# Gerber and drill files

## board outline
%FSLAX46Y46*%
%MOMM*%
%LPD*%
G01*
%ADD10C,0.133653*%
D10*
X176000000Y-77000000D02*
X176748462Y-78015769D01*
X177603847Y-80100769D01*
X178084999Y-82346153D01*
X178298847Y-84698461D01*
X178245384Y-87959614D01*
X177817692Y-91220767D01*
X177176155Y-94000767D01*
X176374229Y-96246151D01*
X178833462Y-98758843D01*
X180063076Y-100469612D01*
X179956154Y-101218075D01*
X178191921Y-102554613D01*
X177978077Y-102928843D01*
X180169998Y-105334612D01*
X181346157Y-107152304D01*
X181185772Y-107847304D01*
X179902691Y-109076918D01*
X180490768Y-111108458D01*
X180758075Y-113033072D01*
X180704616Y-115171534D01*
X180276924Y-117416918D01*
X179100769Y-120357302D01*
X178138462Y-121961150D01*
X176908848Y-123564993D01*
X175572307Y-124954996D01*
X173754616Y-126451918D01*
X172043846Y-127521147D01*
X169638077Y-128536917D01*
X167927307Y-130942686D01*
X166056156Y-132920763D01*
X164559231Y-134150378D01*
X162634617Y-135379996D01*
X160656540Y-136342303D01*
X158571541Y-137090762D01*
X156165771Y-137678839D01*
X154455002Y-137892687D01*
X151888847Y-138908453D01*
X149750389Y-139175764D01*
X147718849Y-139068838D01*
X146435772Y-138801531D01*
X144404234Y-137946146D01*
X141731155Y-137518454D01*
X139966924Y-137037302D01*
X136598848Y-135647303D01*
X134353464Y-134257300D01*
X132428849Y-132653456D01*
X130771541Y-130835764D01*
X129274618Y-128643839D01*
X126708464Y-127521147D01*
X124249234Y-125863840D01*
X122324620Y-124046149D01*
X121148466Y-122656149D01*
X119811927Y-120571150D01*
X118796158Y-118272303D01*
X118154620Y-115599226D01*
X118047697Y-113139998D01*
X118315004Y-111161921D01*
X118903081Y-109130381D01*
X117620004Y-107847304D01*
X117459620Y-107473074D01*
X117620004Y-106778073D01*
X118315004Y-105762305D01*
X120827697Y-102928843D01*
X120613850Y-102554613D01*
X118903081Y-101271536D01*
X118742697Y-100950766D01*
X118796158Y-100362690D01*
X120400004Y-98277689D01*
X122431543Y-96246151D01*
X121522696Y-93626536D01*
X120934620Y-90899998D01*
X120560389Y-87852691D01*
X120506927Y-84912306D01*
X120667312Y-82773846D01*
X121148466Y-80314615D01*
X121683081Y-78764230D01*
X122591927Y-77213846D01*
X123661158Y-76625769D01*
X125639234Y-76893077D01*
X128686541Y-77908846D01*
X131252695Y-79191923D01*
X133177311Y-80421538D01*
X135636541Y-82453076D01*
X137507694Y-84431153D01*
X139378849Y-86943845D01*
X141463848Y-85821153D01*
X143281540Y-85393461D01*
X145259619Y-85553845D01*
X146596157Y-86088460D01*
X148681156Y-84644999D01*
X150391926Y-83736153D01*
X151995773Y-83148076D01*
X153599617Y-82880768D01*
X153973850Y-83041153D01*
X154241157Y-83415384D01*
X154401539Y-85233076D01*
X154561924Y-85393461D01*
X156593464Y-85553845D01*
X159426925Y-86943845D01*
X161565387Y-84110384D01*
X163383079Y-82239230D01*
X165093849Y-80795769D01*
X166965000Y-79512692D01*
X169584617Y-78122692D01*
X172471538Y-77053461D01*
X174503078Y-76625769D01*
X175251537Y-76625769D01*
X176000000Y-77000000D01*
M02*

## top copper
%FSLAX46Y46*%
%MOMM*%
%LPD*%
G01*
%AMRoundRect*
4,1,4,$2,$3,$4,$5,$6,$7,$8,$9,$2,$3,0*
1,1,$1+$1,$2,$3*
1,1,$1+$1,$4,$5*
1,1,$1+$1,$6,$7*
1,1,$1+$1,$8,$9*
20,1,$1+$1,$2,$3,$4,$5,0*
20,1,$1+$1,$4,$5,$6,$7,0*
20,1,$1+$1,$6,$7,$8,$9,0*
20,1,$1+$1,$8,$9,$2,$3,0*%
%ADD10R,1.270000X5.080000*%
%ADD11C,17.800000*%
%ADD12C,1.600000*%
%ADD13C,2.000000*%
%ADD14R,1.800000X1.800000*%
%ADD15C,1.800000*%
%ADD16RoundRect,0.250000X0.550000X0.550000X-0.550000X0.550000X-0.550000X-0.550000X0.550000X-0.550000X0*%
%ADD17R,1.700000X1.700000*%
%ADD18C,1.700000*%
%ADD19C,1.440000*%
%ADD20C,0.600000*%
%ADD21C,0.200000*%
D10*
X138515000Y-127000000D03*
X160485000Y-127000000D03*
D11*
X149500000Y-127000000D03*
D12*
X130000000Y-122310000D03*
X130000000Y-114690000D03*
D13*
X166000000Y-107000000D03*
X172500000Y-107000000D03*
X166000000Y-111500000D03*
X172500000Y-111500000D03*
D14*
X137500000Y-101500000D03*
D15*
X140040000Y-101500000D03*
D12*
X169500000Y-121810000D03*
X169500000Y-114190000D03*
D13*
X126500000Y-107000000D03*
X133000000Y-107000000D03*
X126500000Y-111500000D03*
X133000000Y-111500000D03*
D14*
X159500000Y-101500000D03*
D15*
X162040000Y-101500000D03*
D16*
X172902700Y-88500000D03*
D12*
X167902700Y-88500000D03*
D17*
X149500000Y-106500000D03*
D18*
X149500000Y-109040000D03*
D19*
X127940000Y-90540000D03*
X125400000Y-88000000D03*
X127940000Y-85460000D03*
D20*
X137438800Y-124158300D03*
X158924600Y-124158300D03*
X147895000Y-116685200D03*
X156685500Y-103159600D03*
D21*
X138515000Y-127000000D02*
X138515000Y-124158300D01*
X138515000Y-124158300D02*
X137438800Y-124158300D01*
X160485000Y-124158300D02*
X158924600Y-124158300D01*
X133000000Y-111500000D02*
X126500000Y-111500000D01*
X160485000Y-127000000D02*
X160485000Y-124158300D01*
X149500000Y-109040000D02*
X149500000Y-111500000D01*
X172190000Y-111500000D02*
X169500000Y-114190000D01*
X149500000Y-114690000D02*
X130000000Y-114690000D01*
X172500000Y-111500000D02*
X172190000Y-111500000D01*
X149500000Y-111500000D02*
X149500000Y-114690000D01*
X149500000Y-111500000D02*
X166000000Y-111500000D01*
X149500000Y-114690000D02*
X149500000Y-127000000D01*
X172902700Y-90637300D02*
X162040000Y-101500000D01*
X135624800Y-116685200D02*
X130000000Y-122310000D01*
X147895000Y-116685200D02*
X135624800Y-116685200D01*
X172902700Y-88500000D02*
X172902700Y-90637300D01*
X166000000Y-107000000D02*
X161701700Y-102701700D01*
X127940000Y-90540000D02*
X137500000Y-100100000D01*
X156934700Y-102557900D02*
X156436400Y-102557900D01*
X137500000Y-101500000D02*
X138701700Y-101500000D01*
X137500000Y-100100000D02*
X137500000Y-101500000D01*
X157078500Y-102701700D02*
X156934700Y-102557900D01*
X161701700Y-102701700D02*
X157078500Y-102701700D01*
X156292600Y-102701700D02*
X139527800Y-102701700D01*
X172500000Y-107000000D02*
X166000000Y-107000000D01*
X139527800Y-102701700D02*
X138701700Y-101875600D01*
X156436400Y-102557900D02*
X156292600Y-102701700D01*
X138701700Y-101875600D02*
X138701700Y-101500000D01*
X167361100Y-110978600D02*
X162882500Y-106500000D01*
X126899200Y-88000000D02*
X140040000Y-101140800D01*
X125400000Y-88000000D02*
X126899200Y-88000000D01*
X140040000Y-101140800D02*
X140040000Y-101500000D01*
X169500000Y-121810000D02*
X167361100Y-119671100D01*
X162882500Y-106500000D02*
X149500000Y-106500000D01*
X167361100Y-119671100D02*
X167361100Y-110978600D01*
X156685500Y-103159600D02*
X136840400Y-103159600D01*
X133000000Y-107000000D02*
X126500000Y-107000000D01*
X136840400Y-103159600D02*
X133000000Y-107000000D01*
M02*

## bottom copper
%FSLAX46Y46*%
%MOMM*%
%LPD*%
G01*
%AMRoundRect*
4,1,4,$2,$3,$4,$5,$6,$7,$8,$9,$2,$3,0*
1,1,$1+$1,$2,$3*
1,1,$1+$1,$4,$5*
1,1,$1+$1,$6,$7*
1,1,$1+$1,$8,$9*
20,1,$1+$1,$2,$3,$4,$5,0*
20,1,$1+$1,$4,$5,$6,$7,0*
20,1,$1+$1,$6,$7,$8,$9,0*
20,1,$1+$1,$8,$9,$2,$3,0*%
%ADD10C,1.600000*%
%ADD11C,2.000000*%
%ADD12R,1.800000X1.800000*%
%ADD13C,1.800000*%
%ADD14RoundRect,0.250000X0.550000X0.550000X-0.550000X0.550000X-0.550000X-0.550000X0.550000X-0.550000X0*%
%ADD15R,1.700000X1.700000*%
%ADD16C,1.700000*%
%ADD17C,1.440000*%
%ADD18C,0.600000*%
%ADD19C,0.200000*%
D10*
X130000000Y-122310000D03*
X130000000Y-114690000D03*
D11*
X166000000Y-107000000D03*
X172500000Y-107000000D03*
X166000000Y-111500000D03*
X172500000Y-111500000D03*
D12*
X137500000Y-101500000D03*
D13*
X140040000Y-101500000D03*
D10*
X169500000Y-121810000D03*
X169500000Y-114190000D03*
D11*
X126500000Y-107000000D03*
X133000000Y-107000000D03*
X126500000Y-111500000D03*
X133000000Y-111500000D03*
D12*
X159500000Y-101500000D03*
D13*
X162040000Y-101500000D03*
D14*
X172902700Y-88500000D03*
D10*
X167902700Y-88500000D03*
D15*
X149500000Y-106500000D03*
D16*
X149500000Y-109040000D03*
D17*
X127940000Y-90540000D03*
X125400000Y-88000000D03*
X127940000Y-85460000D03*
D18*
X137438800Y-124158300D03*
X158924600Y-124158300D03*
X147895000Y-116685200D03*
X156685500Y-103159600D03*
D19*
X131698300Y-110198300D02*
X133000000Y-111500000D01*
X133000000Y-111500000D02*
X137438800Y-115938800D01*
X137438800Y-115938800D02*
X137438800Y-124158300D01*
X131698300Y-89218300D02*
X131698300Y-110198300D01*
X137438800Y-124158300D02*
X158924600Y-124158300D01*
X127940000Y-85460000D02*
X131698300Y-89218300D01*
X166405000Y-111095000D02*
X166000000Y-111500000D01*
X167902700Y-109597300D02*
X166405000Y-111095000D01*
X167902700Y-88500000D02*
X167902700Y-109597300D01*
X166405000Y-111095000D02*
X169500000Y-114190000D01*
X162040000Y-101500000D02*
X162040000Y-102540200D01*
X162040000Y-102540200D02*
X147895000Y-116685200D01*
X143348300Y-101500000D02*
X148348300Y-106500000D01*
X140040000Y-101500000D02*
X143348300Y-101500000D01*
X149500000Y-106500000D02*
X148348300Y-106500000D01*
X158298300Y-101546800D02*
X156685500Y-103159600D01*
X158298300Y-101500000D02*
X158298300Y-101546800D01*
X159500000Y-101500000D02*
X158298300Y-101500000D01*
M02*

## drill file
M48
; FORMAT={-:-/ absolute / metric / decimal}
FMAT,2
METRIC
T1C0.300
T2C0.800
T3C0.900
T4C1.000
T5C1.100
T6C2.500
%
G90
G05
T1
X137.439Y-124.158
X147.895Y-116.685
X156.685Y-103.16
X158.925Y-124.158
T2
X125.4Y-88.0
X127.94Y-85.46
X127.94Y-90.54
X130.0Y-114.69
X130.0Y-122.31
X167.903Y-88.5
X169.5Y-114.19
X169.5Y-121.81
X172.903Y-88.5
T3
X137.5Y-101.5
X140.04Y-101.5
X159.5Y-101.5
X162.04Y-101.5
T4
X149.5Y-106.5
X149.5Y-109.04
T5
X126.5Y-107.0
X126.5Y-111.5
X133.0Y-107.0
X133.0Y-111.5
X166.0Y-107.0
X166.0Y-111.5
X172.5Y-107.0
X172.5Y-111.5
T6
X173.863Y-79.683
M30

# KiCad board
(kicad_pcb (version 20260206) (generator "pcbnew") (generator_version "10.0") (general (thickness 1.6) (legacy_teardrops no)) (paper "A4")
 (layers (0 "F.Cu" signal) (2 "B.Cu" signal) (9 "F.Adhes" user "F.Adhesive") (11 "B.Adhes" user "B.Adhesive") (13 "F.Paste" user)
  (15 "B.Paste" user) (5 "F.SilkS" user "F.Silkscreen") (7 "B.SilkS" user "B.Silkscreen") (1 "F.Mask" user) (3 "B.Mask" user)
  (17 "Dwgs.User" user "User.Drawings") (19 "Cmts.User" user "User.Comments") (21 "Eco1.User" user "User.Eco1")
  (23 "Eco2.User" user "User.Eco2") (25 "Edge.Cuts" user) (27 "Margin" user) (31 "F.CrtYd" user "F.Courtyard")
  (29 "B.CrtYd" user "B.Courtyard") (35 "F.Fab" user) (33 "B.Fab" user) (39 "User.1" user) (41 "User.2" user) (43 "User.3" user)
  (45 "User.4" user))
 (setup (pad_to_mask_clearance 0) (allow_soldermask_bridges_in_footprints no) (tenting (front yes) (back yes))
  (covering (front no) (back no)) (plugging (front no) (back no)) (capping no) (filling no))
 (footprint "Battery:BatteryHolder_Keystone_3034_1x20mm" (layer "F.Cu") (at 149.5 127)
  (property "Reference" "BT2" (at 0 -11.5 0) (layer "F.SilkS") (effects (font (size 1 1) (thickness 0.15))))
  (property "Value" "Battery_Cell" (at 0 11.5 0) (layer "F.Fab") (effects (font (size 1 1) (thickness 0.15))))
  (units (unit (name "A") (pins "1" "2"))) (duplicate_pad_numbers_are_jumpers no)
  (pad "1" smd rect (at -10.985 0) (size 1.27 5.08) (layers "F.Cu" "F.Mask" "F.Paste") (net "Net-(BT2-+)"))
  (pad "1" smd rect (at 10.985 0) (size 1.27 5.08) (layers "F.Cu" "F.Mask" "F.Paste") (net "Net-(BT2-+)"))
  (pad "2" smd circle (at 0 0) (size 17.8 17.8) (layers "F.Cu" "F.Mask") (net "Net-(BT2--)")))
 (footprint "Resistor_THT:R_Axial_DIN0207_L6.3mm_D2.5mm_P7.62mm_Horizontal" (layer "F.Cu") (at 130 122.31 90)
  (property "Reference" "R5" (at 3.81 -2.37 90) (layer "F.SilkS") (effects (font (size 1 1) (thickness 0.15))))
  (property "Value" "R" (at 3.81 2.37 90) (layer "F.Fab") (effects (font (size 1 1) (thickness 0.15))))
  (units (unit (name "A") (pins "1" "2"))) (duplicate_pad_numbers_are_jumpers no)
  (pad "1" thru_hole circle (at 0 0 90) (size 1.6 1.6) (drill 0.8) (layers "*.Cu" "*.Mask") (remove_unused_layers no) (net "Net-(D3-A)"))
  (pad "2" thru_hole circle (at 7.62 0 90) (size 1.6 1.6) (drill 0.8) (layers "*.Cu" "*.Mask") (remove_unused_layers no) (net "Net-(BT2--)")))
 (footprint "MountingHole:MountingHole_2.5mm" (layer "F.Cu") (at 173.8631 79.6828)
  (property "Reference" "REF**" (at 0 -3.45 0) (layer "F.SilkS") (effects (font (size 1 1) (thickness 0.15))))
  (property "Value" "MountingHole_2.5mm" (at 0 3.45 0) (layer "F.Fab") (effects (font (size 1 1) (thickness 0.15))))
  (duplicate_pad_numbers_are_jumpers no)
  (pad "" np_thru_hole circle (at 0 0) (size 2.5 2.5) (drill 2.5) (layers "*.Mask")))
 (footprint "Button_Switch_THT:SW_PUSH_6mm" (layer "F.Cu") (at 166 107)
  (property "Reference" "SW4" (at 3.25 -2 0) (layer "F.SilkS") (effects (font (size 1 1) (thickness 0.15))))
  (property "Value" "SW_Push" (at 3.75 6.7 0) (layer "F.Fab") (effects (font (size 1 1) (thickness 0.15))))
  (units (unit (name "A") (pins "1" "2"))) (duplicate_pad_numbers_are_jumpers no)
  (pad "1" thru_hole circle (at 0 0 90) (size 2 2) (drill 1.1) (layers "*.Cu" "*.Mask") (remove_unused_layers no) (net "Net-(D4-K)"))
  (pad "1" thru_hole circle (at 6.5 0 90) (size 2 2) (drill 1.1) (layers "*.Cu" "*.Mask") (remove_unused_layers no) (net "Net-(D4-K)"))
  (pad "2" thru_hole circle (at 0 4.5 90) (size 2 2) (drill 1.1) (layers "*.Cu" "*.Mask") (remove_unused_layers no) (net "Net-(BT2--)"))
  (pad "2" thru_hole circle (at 6.5 4.5 90) (size 2 2) (drill 1.1) (layers "*.Cu" "*.Mask") (remove_unused_layers no) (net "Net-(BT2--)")))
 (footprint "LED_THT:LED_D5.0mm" (layer "F.Cu") (at 137.5 101.5)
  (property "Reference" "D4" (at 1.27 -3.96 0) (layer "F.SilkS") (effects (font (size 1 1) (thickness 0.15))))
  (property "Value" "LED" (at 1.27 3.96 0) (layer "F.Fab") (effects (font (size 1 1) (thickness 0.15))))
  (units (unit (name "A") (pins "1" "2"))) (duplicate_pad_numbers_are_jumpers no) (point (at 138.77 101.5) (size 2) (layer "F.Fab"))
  (pad "1" thru_hole rect (at 0 0) (size 1.8 1.8) (drill 0.9) (layers "*.Cu" "*.Mask") (remove_unused_layers no) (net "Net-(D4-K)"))
  (pad "2" thru_hole circle (at 2.54 0) (size 1.8 1.8) (drill 0.9) (layers "*.Cu" "*.Mask") (remove_unused_layers no) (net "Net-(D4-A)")))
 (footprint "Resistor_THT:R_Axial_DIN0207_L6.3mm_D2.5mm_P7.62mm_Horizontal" (layer "F.Cu") (at 169.5 121.81 90)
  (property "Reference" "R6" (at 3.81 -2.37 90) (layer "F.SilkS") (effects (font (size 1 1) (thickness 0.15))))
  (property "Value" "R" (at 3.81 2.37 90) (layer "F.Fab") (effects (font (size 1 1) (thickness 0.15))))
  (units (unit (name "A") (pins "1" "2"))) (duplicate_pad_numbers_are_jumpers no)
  (pad "1" thru_hole circle (at 0 0 90) (size 1.6 1.6) (drill 0.8) (layers "*.Cu" "*.Mask") (remove_unused_layers no) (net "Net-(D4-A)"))
  (pad "2" thru_hole circle (at 7.62 0 90) (size 1.6 1.6) (drill 0.8) (layers "*.Cu" "*.Mask") (remove_unused_layers no) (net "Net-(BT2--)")))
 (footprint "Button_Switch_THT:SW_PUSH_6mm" (layer "F.Cu") (at 126.5 107)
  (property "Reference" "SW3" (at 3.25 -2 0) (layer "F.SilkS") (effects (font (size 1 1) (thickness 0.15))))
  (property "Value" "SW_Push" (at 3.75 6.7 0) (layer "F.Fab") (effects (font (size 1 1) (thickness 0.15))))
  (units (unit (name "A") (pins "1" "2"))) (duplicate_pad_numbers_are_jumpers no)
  (pad "1" thru_hole circle (at 0 0 90) (size 2 2) (drill 1.1) (layers "*.Cu" "*.Mask") (remove_unused_layers no) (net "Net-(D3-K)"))
  (pad "1" thru_hole circle (at 6.5 0 90) (size 2 2) (drill 1.1) (layers "*.Cu" "*.Mask") (remove_unused_layers no) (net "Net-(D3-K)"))
  (pad "2" thru_hole circle (at 0 4.5 90) (size 2 2) (drill 1.1) (layers "*.Cu" "*.Mask") (remove_unused_layers no) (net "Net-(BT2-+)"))
  (pad "2" thru_hole circle (at 6.5 4.5 90) (size 2 2) (drill 1.1) (layers "*.Cu" "*.Mask") (remove_unused_layers no) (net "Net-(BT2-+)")))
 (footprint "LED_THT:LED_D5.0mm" (layer "F.Cu") (at 159.5 101.5)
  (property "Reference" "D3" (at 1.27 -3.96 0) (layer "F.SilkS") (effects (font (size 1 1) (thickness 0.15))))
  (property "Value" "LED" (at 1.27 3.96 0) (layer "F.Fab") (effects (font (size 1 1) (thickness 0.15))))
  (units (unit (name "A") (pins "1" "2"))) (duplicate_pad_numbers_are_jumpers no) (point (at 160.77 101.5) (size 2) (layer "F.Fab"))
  (pad "1" thru_hole rect (at 0 0) (size 1.8 1.8) (drill 0.9) (layers "*.Cu" "*.Mask") (remove_unused_layers no) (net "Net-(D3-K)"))
  (pad "2" thru_hole circle (at 2.54 0) (size 1.8 1.8) (drill 0.9) (layers "*.Cu" "*.Mask") (remove_unused_layers no) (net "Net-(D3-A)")))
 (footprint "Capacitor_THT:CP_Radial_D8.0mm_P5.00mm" (layer "B.Cu") (at 172.9027 88.5 180)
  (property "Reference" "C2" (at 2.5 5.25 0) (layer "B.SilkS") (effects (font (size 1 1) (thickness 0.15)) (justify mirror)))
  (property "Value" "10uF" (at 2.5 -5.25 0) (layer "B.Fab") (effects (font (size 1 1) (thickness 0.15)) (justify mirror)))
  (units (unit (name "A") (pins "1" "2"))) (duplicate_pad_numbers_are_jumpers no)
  (pad "1" thru_hole roundrect (at 0 0 180) (size 1.6 1.6) (drill 0.8) (layers "*.Cu" "*.Mask") (remove_unused_layers no)
   (roundrect_rratio 0.15625) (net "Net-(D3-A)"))
  (pad "2" thru_hole circle (at 5 0 180) (size 1.6 1.6) (drill 0.8) (layers "*.Cu" "*.Mask") (remove_unused_layers no) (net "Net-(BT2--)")))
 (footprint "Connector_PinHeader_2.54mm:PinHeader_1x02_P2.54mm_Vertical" (layer "B.Cu") (at 149.5 106.5 180)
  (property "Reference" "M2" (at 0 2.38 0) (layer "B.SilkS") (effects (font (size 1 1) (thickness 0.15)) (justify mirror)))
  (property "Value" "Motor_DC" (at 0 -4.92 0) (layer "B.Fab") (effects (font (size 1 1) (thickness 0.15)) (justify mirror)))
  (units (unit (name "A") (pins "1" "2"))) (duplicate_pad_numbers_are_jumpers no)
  (pad "1" thru_hole rect (at 0 0 180) (size 1.7 1.7) (drill 1) (layers "*.Cu" "*.Mask") (remove_unused_layers no) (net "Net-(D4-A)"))
  (pad "2" thru_hole circle (at 0 -2.54 180) (size 1.7 1.7) (drill 1) (layers "*.Cu" "*.Mask") (remove_unused_layers no) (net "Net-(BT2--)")))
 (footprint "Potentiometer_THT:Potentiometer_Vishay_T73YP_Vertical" (layer "B.Cu") (at 127.94 90.54 180)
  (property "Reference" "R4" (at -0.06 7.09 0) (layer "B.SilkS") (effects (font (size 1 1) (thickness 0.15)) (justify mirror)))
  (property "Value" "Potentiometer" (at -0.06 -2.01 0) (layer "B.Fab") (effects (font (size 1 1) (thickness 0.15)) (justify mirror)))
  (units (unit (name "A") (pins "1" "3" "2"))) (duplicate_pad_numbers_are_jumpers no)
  (pad "1" thru_hole circle (at 0 0 180) (size 1.44 1.44) (drill 0.8) (layers "*.Cu" "*.Mask") (remove_unused_layers no) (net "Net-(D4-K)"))
  (pad "2" thru_hole circle (at 2.54 2.54 180) (size 1.44 1.44) (drill 0.8) (layers "*.Cu" "*.Mask") (remove_unused_layers no)
   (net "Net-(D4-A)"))
  (pad "3" thru_hole circle (at 0 5.08 180) (size 1.44 1.44) (drill 0.8) (layers "*.Cu" "*.Mask") (remove_unused_layers no)
   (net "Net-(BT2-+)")))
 (gr_poly
  (pts (xy 176 77) (xy 176.748462 78.015769) (xy 177.603847 80.100769) (xy 178.084999 82.346153) (xy 178.298847 84.698461)
   (xy 178.245384 87.959614) (xy 177.817692 91.220767) (xy 177.176155 94.000767) (xy 176.374229 96.246151) (xy 178.833462 98.758843)
   (xy 180.063076 100.469612) (xy 179.956154 101.218075) (xy 178.191921 102.554613) (xy 177.978077 102.928843) (xy 180.169998 105.334612)
   (xy 181.346157 107.152304) (xy 181.185772 107.847304) (xy 179.902691 109.076918) (xy 180.490768 111.108458) (xy 180.758075 113.033072)
   (xy 180.704616 115.171534) (xy 180.276924 117.416918) (xy 179.100769 120.357302) (xy 178.138462 121.96115) (xy 176.908848 123.564993)
   (xy 175.572307 124.954996) (xy 173.754616 126.451918) (xy 172.043846 127.521147) (xy 169.638077 128.536917) (xy 167.927307 130.942686)
   (xy 166.056156 132.920763) (xy 164.559231 134.150378) (xy 162.634617 135.379996) (xy 160.65654 136.342303) (xy 158.571541 137.090762)
   (xy 156.165771 137.678839) (xy 154.455002 137.892687) (xy 151.888847 138.908453) (xy 149.750389 139.175764) (xy 147.718849 139.068838)
   (xy 146.435772 138.801531) (xy 144.404234 137.946146) (xy 141.731155 137.518454) (xy 139.966924 137.037302) (xy 136.598848 135.647303)
   (xy 134.353464 134.2573) (xy 132.428849 132.653456) (xy 130.771541 130.835764) (xy 129.274618 128.643839) (xy 126.708464 127.521147)
   (xy 124.249234 125.86384) (xy 122.32462 124.046149) (xy 121.148466 122.656149) (xy 119.811927 120.57115) (xy 118.796158 118.272303)
   (xy 118.15462 115.599226) (xy 118.047697 113.139998) (xy 118.315004 111.161921) (xy 118.903081 109.130381) (xy 117.620004 107.847304)
   (xy 117.45962 107.473074) (xy 117.620004 106.778073) (xy 118.315004 105.762305) (xy 120.827697 102.928843) (xy 120.61385 102.554613)
   (xy 118.903081 101.271536) (xy 118.742697 100.950766) (xy 118.796158 100.36269) (xy 120.400004 98.277689) (xy 122.431543 96.246151)
   (xy 121.522696 93.626536) (xy 120.93462 90.899998) (xy 120.560389 87.852691) (xy 120.506927 84.912306) (xy 120.667312 82.773846)
   (xy 121.148466 80.314615) (xy 121.683081 78.76423) (xy 122.591927 77.213846) (xy 123.661158 76.625769) (xy 125.639234 76.893077)
   (xy 128.686541 77.908846) (xy 131.252695 79.191923) (xy 133.177311 80.421538) (xy 135.636541 82.453076) (xy 137.507694 84.431153)
   (xy 139.378849 86.943845) (xy 141.463848 85.821153) (xy 143.28154 85.393461) (xy 145.259619 85.553845) (xy 146.596157 86.08846)
   (xy 148.681156 84.644999) (xy 150.391926 83.736153) (xy 151.995773 83.148076) (xy 153.599617 82.880768) (xy 153.97385 83.041153)
   (xy 154.241157 83.415384) (xy 154.401539 85.233076) (xy 154.561924 85.393461) (xy 156.593464 85.553845) (xy 159.426925 86.943845)
   (xy 161.565387 84.110384) (xy 163.383079 82.23923) (xy 165.093849 80.795769) (xy 166.965 79.512692) (xy 169.584617 78.122692)
   (xy 172.471538 77.053461) (xy 174.503078 76.625769) (xy 175.251537 76.625769))
  (stroke (width 0.133653) (type solid)) (fill no) (layer "Edge.Cuts"))
 (segment (start 138.515 127) (end 138.515 124.1583) (width 0.2) (layer "F.Cu") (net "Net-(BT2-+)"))
 (segment (start 138.515 124.1583) (end 137.4388 124.1583) (width 0.2) (layer "F.Cu") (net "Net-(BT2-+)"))
 (segment (start 160.485 124.1583) (end 158.9246 124.1583) (width 0.2) (layer "F.Cu") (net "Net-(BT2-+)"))
 (segment (start 133 111.5) (end 126.5 111.5) (width 0.2) (layer "F.Cu") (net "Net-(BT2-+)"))
 (segment (start 160.485 127) (end 160.485 124.1583) (width 0.2) (layer "F.Cu") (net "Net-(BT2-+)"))
 (via (at 137.4388 124.1583) (size 0.6) (drill 0.3) (layers "F.Cu" "B.Cu") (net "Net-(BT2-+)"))
 (via (at 158.9246 124.1583) (size 0.6) (drill 0.3) (layers "F.Cu" "B.Cu") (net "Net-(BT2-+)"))
 (segment (start 131.6983 110.1983) (end 133 111.5) (width 0.2) (layer "B.Cu") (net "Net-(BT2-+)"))
 (segment (start 133 111.5) (end 137.4388 115.9388) (width 0.2) (layer "B.Cu") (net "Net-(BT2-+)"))
 (segment (start 137.4388 115.9388) (end 137.4388 124.1583) (width 0.2) (layer "B.Cu") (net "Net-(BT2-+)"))
 (segment (start 131.6983 89.2183) (end 131.6983 110.1983) (width 0.2) (layer "B.Cu") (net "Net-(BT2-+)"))
 (segment (start 137.4388 124.1583) (end 158.9246 124.1583) (width 0.2) (layer "B.Cu") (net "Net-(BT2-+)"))
 (segment (start 127.94 85.46) (end 131.6983 89.2183) (width 0.2) (layer "B.Cu") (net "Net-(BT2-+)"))
 (segment (start 149.5 109.04) (end 149.5 111.5) (width 0.2) (layer "F.Cu") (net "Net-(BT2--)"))
 (segment (start 172.19 111.5) (end 169.5 114.19) (width 0.2) (layer "F.Cu") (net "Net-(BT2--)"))
 (segment (start 149.5 114.69) (end 130 114.69) (width 0.2) (layer "F.Cu") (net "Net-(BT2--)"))
 (segment (start 172.5 111.5) (end 172.19 111.5) (width 0.2) (layer "F.Cu") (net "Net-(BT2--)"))
 (segment (start 149.5 111.5) (end 149.5 114.69) (width 0.2) (layer "F.Cu") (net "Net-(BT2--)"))
 (segment (start 149.5 111.5) (end 166 111.5) (width 0.2) (layer "F.Cu") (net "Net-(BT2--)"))
 (segment (start 149.5 114.69) (end 149.5 127) (width 0.2) (layer "F.Cu") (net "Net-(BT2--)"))
 (segment (start 166.405 111.095) (end 166 111.5) (width 0.2) (layer "B.Cu") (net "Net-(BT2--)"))
 (segment (start 167.9027 109.5973) (end 166.405 111.095) (width 0.2) (layer "B.Cu") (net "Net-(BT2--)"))
 (segment (start 167.9027 88.5) (end 167.9027 109.5973) (width 0.2) (layer "B.Cu") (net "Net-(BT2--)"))
 (segment (start 166.405 111.095) (end 169.5 114.19) (width 0.2) (layer "B.Cu") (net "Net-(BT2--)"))
 (segment (start 172.9027 90.6373) (end 162.04 101.5) (width 0.2) (layer "F.Cu") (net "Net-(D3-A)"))
 (segment (start 135.6248 116.6852) (end 130 122.31) (width 0.2) (layer "F.Cu") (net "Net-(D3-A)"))
 (segment (start 147.895 116.6852) (end 135.6248 116.6852) (width 0.2) (layer "F.Cu") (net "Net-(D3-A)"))
 (segment (start 172.9027 88.5) (end 172.9027 90.6373) (width 0.2) (layer "F.Cu") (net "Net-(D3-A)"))
 (via (at 147.895 116.6852) (size 0.6) (drill 0.3) (layers "F.Cu" "B.Cu") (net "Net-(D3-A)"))
 (segment (start 162.04 101.5) (end 162.04 102.5402) (width 0.2) (layer "B.Cu") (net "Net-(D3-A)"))
 (segment (start 162.04 102.5402) (end 147.895 116.6852) (width 0.2) (layer "B.Cu") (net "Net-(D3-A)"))
 (segment (start 166 107) (end 161.7017 102.7017) (width 0.2) (layer "F.Cu") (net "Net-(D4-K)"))
 (segment (start 127.94 90.54) (end 137.5 100.1) (width 0.2) (layer "F.Cu") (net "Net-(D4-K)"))
 (segment (start 156.9347 102.5579) (end 156.4364 102.5579) (width 0.2) (layer "F.Cu") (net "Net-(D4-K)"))
 (segment (start 137.5 101.5) (end 138.7017 101.5) (width 0.2) (layer "F.Cu") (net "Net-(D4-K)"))
 (segment (start 137.5 100.1) (end 137.5 101.5) (width 0.2) (layer "F.Cu") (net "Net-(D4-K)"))
 (segment (start 157.0785 102.7017) (end 156.9347 102.5579) (width 0.2) (layer "F.Cu") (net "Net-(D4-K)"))
 (segment (start 161.7017 102.7017) (end 157.0785 102.7017) (width 0.2) (layer "F.Cu") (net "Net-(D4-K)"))
 (segment (start 156.2926 102.7017) (end 139.5278 102.7017) (width 0.2) (layer "F.Cu") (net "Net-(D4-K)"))
 (segment (start 172.5 107) (end 166 107) (width 0.2) (layer "F.Cu") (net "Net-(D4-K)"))
 (segment (start 139.5278 102.7017) (end 138.7017 101.8756) (width 0.2) (layer "F.Cu") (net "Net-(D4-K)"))
 (segment (start 156.4364 102.5579) (end 156.2926 102.7017) (width 0.2) (layer "F.Cu") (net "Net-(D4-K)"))
 (segment (start 138.7017 101.8756) (end 138.7017 101.5) (width 0.2) (layer "F.Cu") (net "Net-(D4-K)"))
 (segment (start 167.3611 110.9786) (end 162.8825 106.5) (width 0.2) (layer "F.Cu") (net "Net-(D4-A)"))
 (segment (start 126.8992 88) (end 140.04 101.1408) (width 0.2) (layer "F.Cu") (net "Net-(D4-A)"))
 (segment (start 125.4 88) (end 126.8992 88) (width 0.2) (layer "F.Cu") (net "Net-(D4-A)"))
 (segment (start 140.04 101.1408) (end 140.04 101.5) (width 0.2) (layer "F.Cu") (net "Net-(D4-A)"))
 (segment (start 169.5 121.81) (end 167.3611 119.6711) (width 0.2) (layer "F.Cu") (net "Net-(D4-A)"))
 (segment (start 162.8825 106.5) (end 149.5 106.5) (width 0.2) (layer "F.Cu") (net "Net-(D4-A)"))
 (segment (start 167.3611 119.6711) (end 167.3611 110.9786) (width 0.2) (layer "F.Cu") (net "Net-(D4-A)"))
 (segment (start 143.3483 101.5) (end 148.3483 106.5) (width 0.2) (layer "B.Cu") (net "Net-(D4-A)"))
 (segment (start 140.04 101.5) (end 143.3483 101.5) (width 0.2) (layer "B.Cu") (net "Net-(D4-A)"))
 (segment (start 149.5 106.5) (end 148.3483 106.5) (width 0.2) (layer "B.Cu") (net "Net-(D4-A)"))
 (segment (start 156.6855 103.1596) (end 136.8404 103.1596) (width 0.2) (layer "F.Cu") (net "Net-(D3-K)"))
 (segment (start 133 107) (end 126.5 107) (width 0.2) (layer "F.Cu") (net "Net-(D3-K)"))
 (segment (start 136.8404 103.1596) (end 133 107) (width 0.2) (layer "F.Cu") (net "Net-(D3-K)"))
 (via (at 156.6855 103.1596) (size 0.6) (drill 0.3) (layers "F.Cu" "B.Cu") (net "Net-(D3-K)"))
 (segment (start 158.2983 101.5468) (end 156.6855 103.1596) (width 0.2) (layer "B.Cu") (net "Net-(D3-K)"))
 (segment (start 158.2983 101.5) (end 158.2983 101.5468) (width 0.2) (layer "B.Cu") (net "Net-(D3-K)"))
 (segment (start 159.5 101.5) (end 158.2983 101.5) (width 0.2) (layer "B.Cu") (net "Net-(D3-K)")))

